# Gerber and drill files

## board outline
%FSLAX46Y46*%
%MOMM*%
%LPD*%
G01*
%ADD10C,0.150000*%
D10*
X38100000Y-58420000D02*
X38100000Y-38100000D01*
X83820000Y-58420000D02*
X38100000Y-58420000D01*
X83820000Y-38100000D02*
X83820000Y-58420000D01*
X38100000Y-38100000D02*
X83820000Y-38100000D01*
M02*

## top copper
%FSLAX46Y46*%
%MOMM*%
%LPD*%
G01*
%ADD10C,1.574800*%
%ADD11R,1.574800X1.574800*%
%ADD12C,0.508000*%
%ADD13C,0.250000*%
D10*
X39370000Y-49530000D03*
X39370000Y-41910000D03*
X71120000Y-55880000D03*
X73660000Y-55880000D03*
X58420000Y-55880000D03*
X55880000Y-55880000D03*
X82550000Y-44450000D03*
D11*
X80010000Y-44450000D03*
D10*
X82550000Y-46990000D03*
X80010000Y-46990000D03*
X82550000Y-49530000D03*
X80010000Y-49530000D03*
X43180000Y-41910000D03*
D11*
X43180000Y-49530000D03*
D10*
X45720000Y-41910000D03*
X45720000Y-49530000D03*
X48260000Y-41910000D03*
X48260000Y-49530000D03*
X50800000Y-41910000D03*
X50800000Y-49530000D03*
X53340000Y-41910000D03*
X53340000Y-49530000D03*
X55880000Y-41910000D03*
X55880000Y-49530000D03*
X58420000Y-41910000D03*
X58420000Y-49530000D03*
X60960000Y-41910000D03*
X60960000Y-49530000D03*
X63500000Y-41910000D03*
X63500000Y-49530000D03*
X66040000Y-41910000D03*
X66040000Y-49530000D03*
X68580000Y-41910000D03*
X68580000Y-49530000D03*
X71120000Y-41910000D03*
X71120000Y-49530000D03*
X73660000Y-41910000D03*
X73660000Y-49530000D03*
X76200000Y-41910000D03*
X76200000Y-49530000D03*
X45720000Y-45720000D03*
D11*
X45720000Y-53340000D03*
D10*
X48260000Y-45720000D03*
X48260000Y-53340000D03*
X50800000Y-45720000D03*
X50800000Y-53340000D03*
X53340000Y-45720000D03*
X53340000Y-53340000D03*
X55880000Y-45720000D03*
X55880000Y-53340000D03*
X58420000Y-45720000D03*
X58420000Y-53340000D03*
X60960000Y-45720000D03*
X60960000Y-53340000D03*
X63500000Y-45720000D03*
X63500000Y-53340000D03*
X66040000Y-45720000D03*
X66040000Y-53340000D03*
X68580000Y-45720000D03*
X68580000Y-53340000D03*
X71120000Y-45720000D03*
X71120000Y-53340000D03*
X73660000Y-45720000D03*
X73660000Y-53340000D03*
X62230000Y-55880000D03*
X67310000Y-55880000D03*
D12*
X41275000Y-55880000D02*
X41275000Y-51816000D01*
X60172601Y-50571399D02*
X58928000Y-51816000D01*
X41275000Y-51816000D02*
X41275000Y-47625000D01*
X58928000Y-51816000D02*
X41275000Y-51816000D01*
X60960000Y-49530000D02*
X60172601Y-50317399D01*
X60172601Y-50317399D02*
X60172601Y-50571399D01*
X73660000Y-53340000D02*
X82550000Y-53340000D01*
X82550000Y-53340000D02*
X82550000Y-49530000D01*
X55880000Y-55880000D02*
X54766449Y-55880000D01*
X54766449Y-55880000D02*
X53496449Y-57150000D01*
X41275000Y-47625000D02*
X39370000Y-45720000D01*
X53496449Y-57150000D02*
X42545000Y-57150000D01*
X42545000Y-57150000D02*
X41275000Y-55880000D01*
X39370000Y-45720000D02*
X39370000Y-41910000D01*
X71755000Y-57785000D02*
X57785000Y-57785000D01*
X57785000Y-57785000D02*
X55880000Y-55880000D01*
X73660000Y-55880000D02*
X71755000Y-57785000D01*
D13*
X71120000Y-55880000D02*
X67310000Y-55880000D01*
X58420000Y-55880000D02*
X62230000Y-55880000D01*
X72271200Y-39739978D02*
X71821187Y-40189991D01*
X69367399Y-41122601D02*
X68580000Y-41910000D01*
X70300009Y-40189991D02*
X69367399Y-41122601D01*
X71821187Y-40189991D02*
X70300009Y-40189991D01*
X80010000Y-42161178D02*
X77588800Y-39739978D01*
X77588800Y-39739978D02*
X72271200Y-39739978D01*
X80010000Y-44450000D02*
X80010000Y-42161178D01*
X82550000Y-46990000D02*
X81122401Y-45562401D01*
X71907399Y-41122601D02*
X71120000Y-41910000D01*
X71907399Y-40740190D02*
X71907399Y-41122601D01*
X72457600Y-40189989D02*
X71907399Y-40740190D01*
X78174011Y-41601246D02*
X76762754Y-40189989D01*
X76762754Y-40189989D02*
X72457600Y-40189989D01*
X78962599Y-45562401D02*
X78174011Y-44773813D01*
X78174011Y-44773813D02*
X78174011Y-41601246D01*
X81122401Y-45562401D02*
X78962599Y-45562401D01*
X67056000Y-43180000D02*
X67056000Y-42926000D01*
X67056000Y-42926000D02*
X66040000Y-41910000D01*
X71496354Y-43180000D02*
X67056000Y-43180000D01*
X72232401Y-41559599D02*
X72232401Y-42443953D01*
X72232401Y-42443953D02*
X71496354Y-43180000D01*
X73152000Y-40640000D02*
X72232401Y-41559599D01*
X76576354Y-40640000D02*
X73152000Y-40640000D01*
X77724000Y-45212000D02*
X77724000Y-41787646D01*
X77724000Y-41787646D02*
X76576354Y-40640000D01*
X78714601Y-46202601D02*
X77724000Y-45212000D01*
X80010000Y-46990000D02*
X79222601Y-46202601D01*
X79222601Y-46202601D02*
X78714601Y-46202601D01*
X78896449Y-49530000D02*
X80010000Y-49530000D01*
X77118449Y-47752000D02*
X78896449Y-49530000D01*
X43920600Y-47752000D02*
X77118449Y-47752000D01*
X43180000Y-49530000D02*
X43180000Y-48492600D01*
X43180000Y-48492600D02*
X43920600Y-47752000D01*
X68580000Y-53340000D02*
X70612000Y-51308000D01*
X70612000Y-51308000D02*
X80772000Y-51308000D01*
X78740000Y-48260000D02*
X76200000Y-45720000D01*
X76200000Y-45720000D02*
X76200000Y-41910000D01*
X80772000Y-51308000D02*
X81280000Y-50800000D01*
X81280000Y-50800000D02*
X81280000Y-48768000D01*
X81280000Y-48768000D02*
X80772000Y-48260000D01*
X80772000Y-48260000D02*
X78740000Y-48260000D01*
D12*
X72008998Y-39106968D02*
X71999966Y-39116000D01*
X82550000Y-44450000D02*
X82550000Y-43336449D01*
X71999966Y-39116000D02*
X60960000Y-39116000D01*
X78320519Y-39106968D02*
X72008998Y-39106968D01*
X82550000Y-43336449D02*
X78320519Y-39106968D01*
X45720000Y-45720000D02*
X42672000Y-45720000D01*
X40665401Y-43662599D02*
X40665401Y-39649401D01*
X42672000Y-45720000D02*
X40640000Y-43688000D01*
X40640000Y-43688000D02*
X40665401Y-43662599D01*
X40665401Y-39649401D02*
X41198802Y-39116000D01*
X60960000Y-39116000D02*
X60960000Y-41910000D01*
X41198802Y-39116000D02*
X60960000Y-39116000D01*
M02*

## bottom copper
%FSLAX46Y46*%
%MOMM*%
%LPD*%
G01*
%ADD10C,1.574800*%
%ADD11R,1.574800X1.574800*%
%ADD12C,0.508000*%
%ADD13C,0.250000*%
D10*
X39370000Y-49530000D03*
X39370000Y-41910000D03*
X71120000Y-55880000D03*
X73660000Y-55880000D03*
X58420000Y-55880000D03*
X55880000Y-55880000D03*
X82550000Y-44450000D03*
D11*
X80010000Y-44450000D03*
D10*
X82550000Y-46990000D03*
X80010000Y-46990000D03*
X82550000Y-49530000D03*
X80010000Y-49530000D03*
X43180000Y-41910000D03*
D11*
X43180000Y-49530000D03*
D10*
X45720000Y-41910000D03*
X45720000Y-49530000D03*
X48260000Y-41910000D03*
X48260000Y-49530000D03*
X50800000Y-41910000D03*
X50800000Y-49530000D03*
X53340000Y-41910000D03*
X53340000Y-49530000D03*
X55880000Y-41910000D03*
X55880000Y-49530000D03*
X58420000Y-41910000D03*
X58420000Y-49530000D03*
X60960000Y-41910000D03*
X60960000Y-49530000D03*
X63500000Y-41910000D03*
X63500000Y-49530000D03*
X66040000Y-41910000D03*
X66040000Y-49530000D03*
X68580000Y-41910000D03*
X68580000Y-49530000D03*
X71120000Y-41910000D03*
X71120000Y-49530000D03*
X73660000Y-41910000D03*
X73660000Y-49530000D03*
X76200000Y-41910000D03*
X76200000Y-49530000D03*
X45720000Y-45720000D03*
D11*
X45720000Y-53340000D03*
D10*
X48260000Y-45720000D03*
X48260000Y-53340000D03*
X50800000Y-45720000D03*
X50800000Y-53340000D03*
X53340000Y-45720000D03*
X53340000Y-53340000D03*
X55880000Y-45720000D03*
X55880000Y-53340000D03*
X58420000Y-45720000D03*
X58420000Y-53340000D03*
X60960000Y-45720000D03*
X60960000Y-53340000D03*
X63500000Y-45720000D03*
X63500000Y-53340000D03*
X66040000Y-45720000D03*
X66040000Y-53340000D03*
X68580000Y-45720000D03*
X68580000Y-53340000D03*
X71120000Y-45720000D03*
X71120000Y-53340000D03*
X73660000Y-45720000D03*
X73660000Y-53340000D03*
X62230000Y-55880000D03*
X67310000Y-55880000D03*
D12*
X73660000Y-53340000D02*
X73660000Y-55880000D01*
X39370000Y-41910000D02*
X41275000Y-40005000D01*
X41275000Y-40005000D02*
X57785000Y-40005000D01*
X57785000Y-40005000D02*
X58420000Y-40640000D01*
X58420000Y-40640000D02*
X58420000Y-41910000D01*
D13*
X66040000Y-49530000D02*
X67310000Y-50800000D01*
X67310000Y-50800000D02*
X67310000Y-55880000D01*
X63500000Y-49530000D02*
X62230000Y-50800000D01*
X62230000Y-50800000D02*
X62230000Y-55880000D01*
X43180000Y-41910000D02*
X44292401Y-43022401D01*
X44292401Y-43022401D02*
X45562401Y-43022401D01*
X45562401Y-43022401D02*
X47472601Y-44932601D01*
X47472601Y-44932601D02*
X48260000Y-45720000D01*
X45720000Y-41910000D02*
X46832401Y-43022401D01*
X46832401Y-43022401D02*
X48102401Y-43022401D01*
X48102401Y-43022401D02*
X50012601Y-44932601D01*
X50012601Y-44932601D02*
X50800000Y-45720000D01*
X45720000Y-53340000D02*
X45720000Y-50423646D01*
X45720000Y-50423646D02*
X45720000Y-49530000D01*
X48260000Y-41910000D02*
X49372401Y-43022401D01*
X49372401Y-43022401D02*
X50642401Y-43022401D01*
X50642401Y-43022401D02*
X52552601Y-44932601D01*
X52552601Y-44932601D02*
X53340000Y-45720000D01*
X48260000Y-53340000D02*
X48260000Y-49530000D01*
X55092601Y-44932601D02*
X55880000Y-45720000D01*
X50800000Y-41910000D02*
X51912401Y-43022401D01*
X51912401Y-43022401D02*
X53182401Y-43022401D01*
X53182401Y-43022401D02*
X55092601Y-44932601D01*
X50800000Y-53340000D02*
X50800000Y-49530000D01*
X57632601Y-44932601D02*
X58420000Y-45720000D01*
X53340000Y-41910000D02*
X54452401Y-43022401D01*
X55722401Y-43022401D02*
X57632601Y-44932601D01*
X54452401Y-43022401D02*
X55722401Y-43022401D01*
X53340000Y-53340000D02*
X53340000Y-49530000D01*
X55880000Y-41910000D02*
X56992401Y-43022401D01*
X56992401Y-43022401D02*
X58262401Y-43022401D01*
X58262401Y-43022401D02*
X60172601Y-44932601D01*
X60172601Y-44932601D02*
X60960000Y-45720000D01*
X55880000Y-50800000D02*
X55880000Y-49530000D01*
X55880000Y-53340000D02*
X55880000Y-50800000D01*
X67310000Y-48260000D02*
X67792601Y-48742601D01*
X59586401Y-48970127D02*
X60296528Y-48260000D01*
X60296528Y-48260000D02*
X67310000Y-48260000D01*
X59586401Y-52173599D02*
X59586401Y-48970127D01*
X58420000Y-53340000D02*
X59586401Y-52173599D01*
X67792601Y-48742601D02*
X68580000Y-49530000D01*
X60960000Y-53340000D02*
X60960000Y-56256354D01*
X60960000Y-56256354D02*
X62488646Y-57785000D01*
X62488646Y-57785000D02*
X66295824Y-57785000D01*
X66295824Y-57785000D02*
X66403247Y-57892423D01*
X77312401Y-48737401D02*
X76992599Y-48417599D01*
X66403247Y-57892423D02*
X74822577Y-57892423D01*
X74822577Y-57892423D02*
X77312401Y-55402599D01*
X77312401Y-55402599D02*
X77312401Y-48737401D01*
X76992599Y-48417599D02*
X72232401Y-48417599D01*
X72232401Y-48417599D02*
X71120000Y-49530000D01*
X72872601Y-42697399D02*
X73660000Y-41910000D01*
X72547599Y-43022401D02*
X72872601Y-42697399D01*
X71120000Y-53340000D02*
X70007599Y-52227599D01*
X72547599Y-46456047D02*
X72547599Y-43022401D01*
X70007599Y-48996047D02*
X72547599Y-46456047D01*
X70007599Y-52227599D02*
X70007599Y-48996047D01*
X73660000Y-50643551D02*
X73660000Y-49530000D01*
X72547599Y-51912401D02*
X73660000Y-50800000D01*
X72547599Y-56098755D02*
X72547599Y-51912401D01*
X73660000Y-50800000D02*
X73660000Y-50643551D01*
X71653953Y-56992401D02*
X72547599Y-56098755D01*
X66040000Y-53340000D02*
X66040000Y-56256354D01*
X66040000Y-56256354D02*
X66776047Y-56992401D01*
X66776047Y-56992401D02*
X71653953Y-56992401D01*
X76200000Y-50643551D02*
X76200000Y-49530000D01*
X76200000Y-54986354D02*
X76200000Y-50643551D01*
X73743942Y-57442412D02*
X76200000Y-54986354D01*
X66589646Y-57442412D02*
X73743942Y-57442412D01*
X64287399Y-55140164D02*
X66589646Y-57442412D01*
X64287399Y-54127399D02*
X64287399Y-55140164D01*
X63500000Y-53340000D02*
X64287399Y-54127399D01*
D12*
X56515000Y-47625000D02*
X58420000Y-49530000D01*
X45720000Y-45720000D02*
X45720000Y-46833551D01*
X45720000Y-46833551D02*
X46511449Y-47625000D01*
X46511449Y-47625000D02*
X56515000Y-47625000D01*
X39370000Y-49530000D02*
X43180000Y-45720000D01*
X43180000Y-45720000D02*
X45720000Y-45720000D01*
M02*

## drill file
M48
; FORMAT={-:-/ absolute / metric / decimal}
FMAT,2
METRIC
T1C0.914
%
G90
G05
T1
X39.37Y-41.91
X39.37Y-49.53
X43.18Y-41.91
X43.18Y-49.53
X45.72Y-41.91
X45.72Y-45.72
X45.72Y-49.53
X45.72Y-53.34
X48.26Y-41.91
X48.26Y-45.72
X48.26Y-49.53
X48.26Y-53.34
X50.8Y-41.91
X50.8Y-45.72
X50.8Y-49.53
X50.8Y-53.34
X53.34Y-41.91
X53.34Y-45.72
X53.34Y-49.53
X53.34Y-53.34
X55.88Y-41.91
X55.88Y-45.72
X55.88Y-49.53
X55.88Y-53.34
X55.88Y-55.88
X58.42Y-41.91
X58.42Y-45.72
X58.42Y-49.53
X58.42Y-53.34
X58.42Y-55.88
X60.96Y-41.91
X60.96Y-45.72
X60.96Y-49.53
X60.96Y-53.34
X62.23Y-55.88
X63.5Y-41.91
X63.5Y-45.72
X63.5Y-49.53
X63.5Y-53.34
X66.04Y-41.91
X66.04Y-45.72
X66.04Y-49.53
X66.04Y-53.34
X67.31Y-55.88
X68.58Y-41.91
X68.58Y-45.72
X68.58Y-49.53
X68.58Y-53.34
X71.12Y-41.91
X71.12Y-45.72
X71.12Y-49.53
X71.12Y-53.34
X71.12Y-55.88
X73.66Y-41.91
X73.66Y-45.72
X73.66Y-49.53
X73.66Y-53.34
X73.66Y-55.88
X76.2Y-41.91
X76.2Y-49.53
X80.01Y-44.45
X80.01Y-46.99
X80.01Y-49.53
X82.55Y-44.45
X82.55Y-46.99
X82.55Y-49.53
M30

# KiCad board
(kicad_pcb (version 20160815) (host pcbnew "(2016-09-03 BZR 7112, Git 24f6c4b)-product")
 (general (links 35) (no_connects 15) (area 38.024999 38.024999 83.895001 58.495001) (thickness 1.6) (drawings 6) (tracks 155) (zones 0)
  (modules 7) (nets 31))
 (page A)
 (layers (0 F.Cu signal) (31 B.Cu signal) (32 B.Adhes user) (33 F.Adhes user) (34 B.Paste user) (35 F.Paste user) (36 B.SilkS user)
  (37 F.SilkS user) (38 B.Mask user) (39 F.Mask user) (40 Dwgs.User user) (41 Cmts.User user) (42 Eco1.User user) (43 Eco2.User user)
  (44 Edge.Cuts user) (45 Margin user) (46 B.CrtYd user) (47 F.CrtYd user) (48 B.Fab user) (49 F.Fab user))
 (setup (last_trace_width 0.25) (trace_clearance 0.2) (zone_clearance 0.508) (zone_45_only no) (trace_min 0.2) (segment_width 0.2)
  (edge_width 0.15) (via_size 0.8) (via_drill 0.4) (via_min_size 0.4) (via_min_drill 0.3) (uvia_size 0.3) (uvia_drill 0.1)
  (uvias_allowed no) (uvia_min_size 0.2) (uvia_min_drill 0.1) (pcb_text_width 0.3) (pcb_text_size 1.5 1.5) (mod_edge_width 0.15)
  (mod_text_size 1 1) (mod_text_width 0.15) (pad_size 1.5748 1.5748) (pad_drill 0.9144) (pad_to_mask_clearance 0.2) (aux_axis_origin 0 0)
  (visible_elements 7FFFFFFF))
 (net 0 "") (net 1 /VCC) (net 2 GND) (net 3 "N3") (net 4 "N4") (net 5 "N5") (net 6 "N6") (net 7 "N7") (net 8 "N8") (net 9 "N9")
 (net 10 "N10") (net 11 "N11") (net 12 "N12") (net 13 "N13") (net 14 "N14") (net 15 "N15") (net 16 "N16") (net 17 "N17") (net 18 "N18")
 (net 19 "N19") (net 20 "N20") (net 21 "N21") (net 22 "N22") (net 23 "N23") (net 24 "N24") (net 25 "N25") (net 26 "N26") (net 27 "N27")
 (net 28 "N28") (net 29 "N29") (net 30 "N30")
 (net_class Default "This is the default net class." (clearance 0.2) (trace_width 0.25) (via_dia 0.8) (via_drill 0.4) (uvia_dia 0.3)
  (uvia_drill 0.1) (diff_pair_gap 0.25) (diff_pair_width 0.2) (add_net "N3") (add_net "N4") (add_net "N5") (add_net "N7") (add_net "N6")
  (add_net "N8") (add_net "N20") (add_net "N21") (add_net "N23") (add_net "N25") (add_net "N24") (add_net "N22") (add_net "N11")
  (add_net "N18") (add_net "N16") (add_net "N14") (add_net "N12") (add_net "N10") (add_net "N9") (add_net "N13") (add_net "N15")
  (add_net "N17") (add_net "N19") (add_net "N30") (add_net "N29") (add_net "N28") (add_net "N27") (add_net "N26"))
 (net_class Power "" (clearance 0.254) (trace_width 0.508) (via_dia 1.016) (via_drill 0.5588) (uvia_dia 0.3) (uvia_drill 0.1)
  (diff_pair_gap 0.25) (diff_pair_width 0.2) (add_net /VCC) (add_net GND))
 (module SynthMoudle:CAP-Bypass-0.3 (layer F.Cu) (at 39.37 45.72 90)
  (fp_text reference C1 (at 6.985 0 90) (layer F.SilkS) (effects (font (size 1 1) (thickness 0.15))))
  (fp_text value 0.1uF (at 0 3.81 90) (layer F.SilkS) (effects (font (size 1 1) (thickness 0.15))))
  (pad 1 thru_hole circle (at -3.81 0 90) (size 1.5748 1.5748) (drill 0.9144) (layers *.Cu *.Mask F.SilkS) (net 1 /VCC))
  (pad 2 thru_hole circle (at 3.81 0 90) (size 1.5748 1.5748) (drill 0.9144) (layers *.Cu *.Mask F.SilkS) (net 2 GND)))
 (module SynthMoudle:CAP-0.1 (layer F.Cu) (at 72.39 55.88)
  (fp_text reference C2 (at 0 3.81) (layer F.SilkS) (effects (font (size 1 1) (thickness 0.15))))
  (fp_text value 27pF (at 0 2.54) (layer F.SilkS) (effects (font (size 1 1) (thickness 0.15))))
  (pad 1 thru_hole circle (at -1.27 0) (size 1.5748 1.5748) (drill 0.9144) (layers *.Cu *.Mask F.SilkS) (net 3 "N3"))
  (pad 2 thru_hole circle (at 1.27 0) (size 1.5748 1.5748) (drill 0.9144) (layers *.Cu *.Mask F.SilkS) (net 2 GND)))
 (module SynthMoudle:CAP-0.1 (layer F.Cu) (at 57.15 55.88 180)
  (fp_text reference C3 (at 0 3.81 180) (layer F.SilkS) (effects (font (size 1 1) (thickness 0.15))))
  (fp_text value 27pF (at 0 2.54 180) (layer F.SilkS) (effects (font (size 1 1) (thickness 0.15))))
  (pad 1 thru_hole circle (at -1.27 0 180) (size 1.5748 1.5748) (drill 0.9144) (layers *.Cu *.Mask F.SilkS) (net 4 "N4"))
  (pad 2 thru_hole circle (at 1.27 0 180) (size 1.5748 1.5748) (drill 0.9144) (layers *.Cu *.Mask F.SilkS) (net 2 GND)))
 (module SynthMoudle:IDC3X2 (layer F.Cu) (at 81.28 46.99 270)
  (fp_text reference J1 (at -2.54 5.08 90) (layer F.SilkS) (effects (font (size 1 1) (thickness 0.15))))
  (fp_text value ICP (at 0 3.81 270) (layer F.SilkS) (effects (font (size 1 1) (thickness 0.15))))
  (pad 2 thru_hole circle (at -2.54 -1.27 270) (size 1.5748 1.5748) (drill 0.9144) (layers *.Cu *.Mask) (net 1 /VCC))
  (pad 1 thru_hole rect (at -2.54 1.27 270) (size 1.5748 1.5748) (drill 0.9144) (layers *.Cu *.Mask) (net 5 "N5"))
  (pad 4 thru_hole circle (at 0 -1.27 270) (size 1.5748 1.5748) (drill 0.9144) (layers *.Cu *.Mask) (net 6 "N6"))
  (pad 3 thru_hole circle (at 0 1.27 270) (size 1.5748 1.5748) (drill 0.9144) (layers *.Cu *.Mask) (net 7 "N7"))
  (pad 6 thru_hole circle (at 2.54 -1.27 270) (size 1.5748 1.5748) (drill 0.9144) (layers *.Cu *.Mask) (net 2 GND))
  (pad 5 thru_hole circle (at 2.54 1.27 270) (size 1.5748 1.5748) (drill 0.9144) (layers *.Cu *.Mask) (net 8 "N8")))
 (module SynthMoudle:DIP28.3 (layer F.Cu) (at 59.69 45.72)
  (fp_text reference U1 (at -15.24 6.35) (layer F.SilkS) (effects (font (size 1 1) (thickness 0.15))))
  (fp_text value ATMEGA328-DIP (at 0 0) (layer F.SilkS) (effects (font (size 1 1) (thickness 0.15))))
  (pad 28 thru_hole circle (at -16.51 -3.81) (size 1.5748 1.5748) (drill 0.9144) (layers *.Cu *.Mask) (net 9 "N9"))
  (pad 1 thru_hole rect (at -16.51 3.81) (size 1.5748 1.5748) (drill 0.9144) (layers *.Cu *.Mask) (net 8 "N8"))
  (pad 27 thru_hole circle (at -13.97 -3.81) (size 1.5748 1.5748) (drill 0.9144) (layers *.Cu *.Mask) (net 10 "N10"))
  (pad 2 thru_hole circle (at -13.97 3.81) (size 1.5748 1.5748) (drill 0.9144) (layers *.Cu *.Mask) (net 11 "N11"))
  (pad 26 thru_hole circle (at -11.43 -3.81) (size 1.5748 1.5748) (drill 0.9144) (layers *.Cu *.Mask) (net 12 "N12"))
  (pad 3 thru_hole circle (at -11.43 3.81) (size 1.5748 1.5748) (drill 0.9144) (layers *.Cu *.Mask) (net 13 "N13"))
  (pad 25 thru_hole circle (at -8.89 -3.81) (size 1.5748 1.5748) (drill 0.9144) (layers *.Cu *.Mask) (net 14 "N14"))
  (pad 4 thru_hole circle (at -8.89 3.81) (size 1.5748 1.5748) (drill 0.9144) (layers *.Cu *.Mask) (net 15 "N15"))
  (pad 24 thru_hole circle (at -6.35 -3.81) (size 1.5748 1.5748) (drill 0.9144) (layers *.Cu *.Mask) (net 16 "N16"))
  (pad 5 thru_hole circle (at -6.35 3.81) (size 1.5748 1.5748) (drill 0.9144) (layers *.Cu *.Mask) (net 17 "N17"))
  (pad 23 thru_hole circle (at -3.81 -3.81) (size 1.5748 1.5748) (drill 0.9144) (layers *.Cu *.Mask) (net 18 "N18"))
  (pad 6 thru_hole circle (at -3.81 3.81) (size 1.5748 1.5748) (drill 0.9144) (layers *.Cu *.Mask) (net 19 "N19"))
  (pad 22 thru_hole circle (at -1.27 -3.81) (size 1.5748 1.5748) (drill 0.9144) (layers *.Cu *.Mask) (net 2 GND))
  (pad 7 thru_hole circle (at -1.27 3.81) (size 1.5748 1.5748) (drill 0.9144) (layers *.Cu *.Mask) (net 1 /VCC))
  (pad 21 thru_hole circle (at 1.27 -3.81) (size 1.5748 1.5748) (drill 0.9144) (layers *.Cu *.Mask) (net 1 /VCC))
  (pad 8 thru_hole circle (at 1.27 3.81) (size 1.5748 1.5748) (drill 0.9144) (layers *.Cu *.Mask) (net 2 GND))
  (pad 20 thru_hole circle (at 3.81 -3.81) (size 1.5748 1.5748) (drill 0.9144) (layers *.Cu *.Mask))
  (pad 9 thru_hole circle (at 3.81 3.81) (size 1.5748 1.5748) (drill 0.9144) (layers *.Cu *.Mask) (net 4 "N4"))
  (pad 19 thru_hole circle (at 6.35 -3.81) (size 1.5748 1.5748) (drill 0.9144) (layers *.Cu *.Mask) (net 7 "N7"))
  (pad 10 thru_hole circle (at 6.35 3.81) (size 1.5748 1.5748) (drill 0.9144) (layers *.Cu *.Mask) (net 3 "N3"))
  (pad 18 thru_hole circle (at 8.89 -3.81) (size 1.5748 1.5748) (drill 0.9144) (layers *.Cu *.Mask) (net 5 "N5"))
  (pad 11 thru_hole circle (at 8.89 3.81) (size 1.5748 1.5748) (drill 0.9144) (layers *.Cu *.Mask) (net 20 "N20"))
  (pad 17 thru_hole circle (at 11.43 -3.81) (size 1.5748 1.5748) (drill 0.9144) (layers *.Cu *.Mask) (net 6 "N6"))
  (pad 12 thru_hole circle (at 11.43 3.81) (size 1.5748 1.5748) (drill 0.9144) (layers *.Cu *.Mask) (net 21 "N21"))
  (pad 16 thru_hole circle (at 13.97 -3.81) (size 1.5748 1.5748) (drill 0.9144) (layers *.Cu *.Mask) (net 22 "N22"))
  (pad 13 thru_hole circle (at 13.97 3.81) (size 1.5748 1.5748) (drill 0.9144) (layers *.Cu *.Mask) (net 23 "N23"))
  (pad 15 thru_hole circle (at 16.51 -3.81) (size 1.5748 1.5748) (drill 0.9144) (layers *.Cu *.Mask) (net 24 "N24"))
  (pad 14 thru_hole circle (at 16.51 3.81) (size 1.5748 1.5748) (drill 0.9144) (layers *.Cu *.Mask) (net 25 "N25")))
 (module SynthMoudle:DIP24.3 (layer F.Cu) (at 59.69 49.53)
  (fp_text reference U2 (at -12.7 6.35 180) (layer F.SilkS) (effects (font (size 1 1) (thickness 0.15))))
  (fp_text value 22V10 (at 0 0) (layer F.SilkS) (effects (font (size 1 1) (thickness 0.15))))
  (pad 24 thru_hole circle (at -13.97 -3.81) (size 1.5748 1.5748) (drill 0.9144) (layers *.Cu *.Mask) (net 1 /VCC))
  (pad 1 thru_hole rect (at -13.97 3.81) (size 1.5748 1.5748) (drill 0.9144) (layers *.Cu *.Mask) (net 11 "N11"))
  (pad 23 thru_hole circle (at -11.43 -3.81) (size 1.5748 1.5748) (drill 0.9144) (layers *.Cu *.Mask) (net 9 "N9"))
  (pad 2 thru_hole circle (at -11.43 3.81) (size 1.5748 1.5748) (drill 0.9144) (layers *.Cu *.Mask) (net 13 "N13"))
  (pad 22 thru_hole circle (at -8.89 -3.81) (size 1.5748 1.5748) (drill 0.9144) (layers *.Cu *.Mask) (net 10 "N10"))
  (pad 3 thru_hole circle (at -8.89 3.81) (size 1.5748 1.5748) (drill 0.9144) (layers *.Cu *.Mask) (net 15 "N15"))
  (pad 21 thru_hole circle (at -6.35 -3.81) (size 1.5748 1.5748) (drill 0.9144) (layers *.Cu *.Mask) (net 12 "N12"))
  (pad 4 thru_hole circle (at -6.35 3.81) (size 1.5748 1.5748) (drill 0.9144) (layers *.Cu *.Mask) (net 17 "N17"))
  (pad 20 thru_hole circle (at -3.81 -3.81) (size 1.5748 1.5748) (drill 0.9144) (layers *.Cu *.Mask) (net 14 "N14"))
  (pad 5 thru_hole circle (at -3.81 3.81) (size 1.5748 1.5748) (drill 0.9144) (layers *.Cu *.Mask) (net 19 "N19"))
  (pad 19 thru_hole circle (at -1.27 -3.81) (size 1.5748 1.5748) (drill 0.9144) (layers *.Cu *.Mask) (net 16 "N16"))
  (pad 6 thru_hole circle (at -1.27 3.81) (size 1.5748 1.5748) (drill 0.9144) (layers *.Cu *.Mask) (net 20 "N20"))
  (pad 18 thru_hole circle (at 1.27 -3.81) (size 1.5748 1.5748) (drill 0.9144) (layers *.Cu *.Mask) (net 18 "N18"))
  (pad 7 thru_hole circle (at 1.27 3.81) (size 1.5748 1.5748) (drill 0.9144) (layers *.Cu *.Mask) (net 21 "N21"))
  (pad 17 thru_hole circle (at 3.81 -3.81) (size 1.5748 1.5748) (drill 0.9144) (layers *.Cu *.Mask) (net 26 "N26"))
  (pad 8 thru_hole circle (at 3.81 3.81) (size 1.5748 1.5748) (drill 0.9144) (layers *.Cu *.Mask) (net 25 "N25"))
  (pad 16 thru_hole circle (at 6.35 -3.81) (size 1.5748 1.5748) (drill 0.9144) (layers *.Cu *.Mask) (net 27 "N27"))
  (pad 9 thru_hole circle (at 6.35 3.81) (size 1.5748 1.5748) (drill 0.9144) (layers *.Cu *.Mask) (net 23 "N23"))
  (pad 15 thru_hole circle (at 8.89 -3.81) (size 1.5748 1.5748) (drill 0.9144) (layers *.Cu *.Mask) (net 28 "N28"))
  (pad 10 thru_hole circle (at 8.89 3.81) (size 1.5748 1.5748) (drill 0.9144) (layers *.Cu *.Mask) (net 24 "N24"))
  (pad 14 thru_hole circle (at 11.43 -3.81) (size 1.5748 1.5748) (drill 0.9144) (layers *.Cu *.Mask) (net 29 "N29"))
  (pad 11 thru_hole circle (at 11.43 3.81) (size 1.5748 1.5748) (drill 0.9144) (layers *.Cu *.Mask) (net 22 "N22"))
  (pad 13 thru_hole circle (at 13.97 -3.81) (size 1.5748 1.5748) (drill 0.9144) (layers *.Cu *.Mask) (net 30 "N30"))
  (pad 12 thru_hole circle (at 13.97 3.81) (size 1.5748 1.5748) (drill 0.9144) (layers *.Cu *.Mask) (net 2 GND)))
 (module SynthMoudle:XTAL (layer F.Cu) (at 64.77 55.88)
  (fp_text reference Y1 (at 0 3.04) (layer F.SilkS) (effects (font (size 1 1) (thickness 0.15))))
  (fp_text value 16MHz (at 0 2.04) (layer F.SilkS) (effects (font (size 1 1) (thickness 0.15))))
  (pad 1 thru_hole circle (at -2.54 0) (size 1.5748 1.5748) (drill 0.9144) (layers *.Cu *.Mask F.SilkS) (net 4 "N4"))
  (pad 2 thru_hole circle (at 2.54 0) (size 1.5748 1.5748) (drill 0.9144) (layers *.Cu *.Mask F.SilkS) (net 3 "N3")))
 (gr_line (start 38.1 58.42) (end 38.1 38.1) (angle 90) (layer Edge.Cuts) (width 0.15))
 (gr_line (start 83.82 58.42) (end 38.1 58.42) (angle 90) (layer Edge.Cuts) (width 0.15))
 (gr_line (start 83.82 38.1) (end 83.82 58.42) (angle 90) (layer Edge.Cuts) (width 0.15))
 (gr_line (start 38.1 38.1) (end 83.82 38.1) (angle 90) (layer Edge.Cuts) (width 0.15))
 (segment (start 41.275 55.88) (end 41.275 51.816) (width 0.508) (layer F.Cu) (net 2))
 (segment (start 60.172601 50.571399) (end 58.928 51.816) (width 0.508) (layer F.Cu) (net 2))
 (segment (start 41.275 51.816) (end 41.275 47.625) (width 0.508) (layer F.Cu) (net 2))
 (segment (start 58.928 51.816) (end 41.275 51.816) (width 0.508) (layer F.Cu) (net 2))
 (segment (start 60.96 49.53) (end 60.172601 50.317399) (width 0.508) (layer F.Cu) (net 2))
 (segment (start 60.172601 50.317399) (end 60.172601 50.571399) (width 0.508) (layer F.Cu) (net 2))
 (segment (start 73.66 53.34) (end 82.55 53.34) (width 0.508) (layer F.Cu) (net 2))
 (segment (start 82.55 53.34) (end 82.55 49.53) (width 0.508) (layer F.Cu) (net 2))
 (segment (start 55.88 55.88) (end 54.766449 55.88) (width 0.508) (layer F.Cu) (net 2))
 (segment (start 54.766449 55.88) (end 53.496449 57.15) (width 0.508) (layer F.Cu) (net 2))
 (segment (start 41.275 47.625) (end 39.37 45.72) (width 0.508) (layer F.Cu) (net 2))
 (segment (start 53.496449 57.15) (end 42.545 57.15) (width 0.508) (layer F.Cu) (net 2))
 (segment (start 42.545 57.15) (end 41.275 55.88) (width 0.508) (layer F.Cu) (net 2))
 (segment (start 39.37 45.72) (end 39.37 41.91) (width 0.508) (layer F.Cu) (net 2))
 (segment (start 71.755 57.785) (end 57.785 57.785) (width 0.508) (layer F.Cu) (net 2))
 (segment (start 57.785 57.785) (end 55.88 55.88) (width 0.508) (layer F.Cu) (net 2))
 (segment (start 73.66 55.88) (end 71.755 57.785) (width 0.508) (layer F.Cu) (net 2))
 (segment (start 73.66 53.34) (end 73.66 55.88) (width 0.508) (layer B.Cu) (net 2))
 (segment (start 39.37 41.91) (end 41.275 40.005) (width 0.508) (layer B.Cu) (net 2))
 (segment (start 41.275 40.005) (end 57.785 40.005) (width 0.508) (layer B.Cu) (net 2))
 (segment (start 57.785 40.005) (end 58.42 40.64) (width 0.508) (layer B.Cu) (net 2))
 (segment (start 58.42 40.64) (end 58.42 41.91) (width 0.508) (layer B.Cu) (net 2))
 (segment (start 66.04 49.53) (end 67.31 50.8) (width 0.25) (layer B.Cu) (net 3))
 (segment (start 67.31 50.8) (end 67.31 55.88) (width 0.25) (layer B.Cu) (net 3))
 (segment (start 71.12 55.88) (end 67.31 55.88) (width 0.25) (layer F.Cu) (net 3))
 (segment (start 63.5 49.53) (end 62.23 50.8) (width 0.25) (layer B.Cu) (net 4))
 (segment (start 62.23 50.8) (end 62.23 55.88) (width 0.25) (layer B.Cu) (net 4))
 (segment (start 58.42 55.88) (end 62.23 55.88) (width 0.25) (layer F.Cu) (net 4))
 (segment (start 72.2712 39.739978) (end 71.821187 40.189991) (width 0.25) (layer F.Cu) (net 5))
 (segment (start 69.367399 41.122601) (end 68.58 41.91) (width 0.25) (layer F.Cu) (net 5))
 (segment (start 70.300009 40.189991) (end 69.367399 41.122601) (width 0.25) (layer F.Cu) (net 5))
 (segment (start 71.821187 40.189991) (end 70.300009 40.189991) (width 0.25) (layer F.Cu) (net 5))
 (segment (start 80.01 42.161178) (end 77.5888 39.739978) (width 0.25) (layer F.Cu) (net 5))
 (segment (start 77.5888 39.739978) (end 72.2712 39.739978) (width 0.25) (layer F.Cu) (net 5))
 (segment (start 80.01 44.45) (end 80.01 42.161178) (width 0.25) (layer F.Cu) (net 5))
 (segment (start 82.55 46.99) (end 81.122401 45.562401) (width 0.25) (layer F.Cu) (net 6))
 (segment (start 71.907399 41.122601) (end 71.12 41.91) (width 0.25) (layer F.Cu) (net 6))
 (segment (start 71.907399 40.74019) (end 71.907399 41.122601) (width 0.25) (layer F.Cu) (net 6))
 (segment (start 72.4576 40.189989) (end 71.907399 40.74019) (width 0.25) (layer F.Cu) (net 6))
 (segment (start 78.174011 41.601246) (end 76.762754 40.189989) (width 0.25) (layer F.Cu) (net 6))
 (segment (start 76.762754 40.189989) (end 72.4576 40.189989) (width 0.25) (layer F.Cu) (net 6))
 (segment (start 78.962599 45.562401) (end 78.174011 44.773813) (width 0.25) (layer F.Cu) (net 6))
 (segment (start 78.174011 44.773813) (end 78.174011 41.601246) (width 0.25) (layer F.Cu) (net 6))
 (segment (start 81.122401 45.562401) (end 78.962599 45.562401) (width 0.25) (layer F.Cu) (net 6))
 (segment (start 67.056 43.18) (end 67.056 42.926) (width 0.25) (layer F.Cu) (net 7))
 (segment (start 67.056 42.926) (end 66.04 41.91) (width 0.25) (layer F.Cu) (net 7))
 (segment (start 71.496354 43.18) (end 67.056 43.18) (width 0.25) (layer F.Cu) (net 7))
 (segment (start 72.232401 41.559599) (end 72.232401 42.443953) (width 0.25) (layer F.Cu) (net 7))
 (segment (start 72.232401 42.443953) (end 71.496354 43.18) (width 0.25) (layer F.Cu) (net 7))
 (segment (start 73.152 40.64) (end 72.232401 41.559599) (width 0.25) (layer F.Cu) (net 7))
 (segment (start 76.576354 40.64) (end 73.152 40.64) (width 0.25) (layer F.Cu) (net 7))
 (segment (start 77.724 45.212) (end 77.724 41.787646) (width 0.25) (layer F.Cu) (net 7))
 (segment (start 77.724 41.787646) (end 76.576354 40.64) (width 0.25) (layer F.Cu) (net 7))
 (segment (start 78.714601 46.202601) (end 77.724 45.212) (width 0.25) (layer F.Cu) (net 7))
 (segment (start 80.01 46.99) (end 79.222601 46.202601) (width 0.25) (layer F.Cu) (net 7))
 (segment (start 79.222601 46.202601) (end 78.714601 46.202601) (width 0.25) (layer F.Cu) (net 7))
 (segment (start 78.896449 49.53) (end 80.01 49.53) (width 0.25) (layer F.Cu) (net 8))
 (segment (start 77.118449 47.752) (end 78.896449 49.53) (width 0.25) (layer F.Cu) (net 8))
 (segment (start 43.9206 47.752) (end 77.118449 47.752) (width 0.25) (layer F.Cu) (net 8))
 (segment (start 43.18 49.53) (end 43.18 48.4926) (width 0.25) (layer F.Cu) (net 8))
 (segment (start 43.18 48.4926) (end 43.9206 47.752) (width 0.25) (layer F.Cu) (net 8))
 (segment (start 43.18 41.91) (end 44.292401 43.022401) (width 0.25) (layer B.Cu) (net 9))
 (segment (start 44.292401 43.022401) (end 45.562401 43.022401) (width 0.25) (layer B.Cu) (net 9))
 (segment (start 45.562401 43.022401) (end 47.472601 44.932601) (width 0.25) (layer B.Cu) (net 9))
 (segment (start 47.472601 44.932601) (end 48.26 45.72) (width 0.25) (layer B.Cu) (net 9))
 (segment (start 45.72 41.91) (end 46.832401 43.022401) (width 0.25) (layer B.Cu) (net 10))
 (segment (start 46.832401 43.022401) (end 48.102401 43.022401) (width 0.25) (layer B.Cu) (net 10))
 (segment (start 48.102401 43.022401) (end 50.012601 44.932601) (width 0.25) (layer B.Cu) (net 10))
 (segment (start 50.012601 44.932601) (end 50.8 45.72) (width 0.25) (layer B.Cu) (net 10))
 (segment (start 45.72 53.34) (end 45.72 50.423646) (width 0.25) (layer B.Cu) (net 11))
 (segment (start 45.72 50.423646) (end 45.72 49.53) (width 0.25) (layer B.Cu) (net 11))
 (segment (start 48.26 41.91) (end 49.372401 43.022401) (width 0.25) (layer B.Cu) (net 12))
 (segment (start 49.372401 43.022401) (end 50.642401 43.022401) (width 0.25) (layer B.Cu) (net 12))
 (segment (start 50.642401 43.022401) (end 52.552601 44.932601) (width 0.25) (layer B.Cu) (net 12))
 (segment (start 52.552601 44.932601) (end 53.34 45.72) (width 0.25) (layer B.Cu) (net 12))
 (segment (start 48.26 53.34) (end 48.26 49.53) (width 0.25) (layer B.Cu) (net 13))
 (segment (start 55.092601 44.932601) (end 55.88 45.72) (width 0.25) (layer B.Cu) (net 14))
 (segment (start 50.8 41.91) (end 51.912401 43.022401) (width 0.25) (layer B.Cu) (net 14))
 (segment (start 51.912401 43.022401) (end 53.182401 43.022401) (width 0.25) (layer B.Cu) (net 14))
 (segment (start 53.182401 43.022401) (end 55.092601 44.932601) (width 0.25) (layer B.Cu) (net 14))
 (segment (start 50.8 53.34) (end 50.8 49.53) (width 0.25) (layer B.Cu) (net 15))
 (segment (start 57.632601 44.932601) (end 58.42 45.72) (width 0.25) (layer B.Cu) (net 16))
 (segment (start 53.34 41.91) (end 54.452401 43.022401) (width 0.25) (layer B.Cu) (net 16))
 (segment (start 55.722401 43.022401) (end 57.632601 44.932601) (width 0.25) (layer B.Cu) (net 16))
 (segment (start 54.452401 43.022401) (end 55.722401 43.022401) (width 0.25) (layer B.Cu) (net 16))
 (segment (start 53.34 53.34) (end 53.34 49.53) (width 0.25) (layer B.Cu) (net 17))
 (segment (start 55.88 41.91) (end 56.992401 43.022401) (width 0.25) (layer B.Cu) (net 18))
 (segment (start 56.992401 43.022401) (end 58.262401 43.022401) (width 0.25) (layer B.Cu) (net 18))
 (segment (start 58.262401 43.022401) (end 60.172601 44.932601) (width 0.25) (layer B.Cu) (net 18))
 (segment (start 60.172601 44.932601) (end 60.96 45.72) (width 0.25) (layer B.Cu) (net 18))
 (segment (start 55.88 50.8) (end 55.88 49.53) (width 0.25) (layer B.Cu) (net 19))
 (segment (start 55.88 53.34) (end 55.88 50.8) (width 0.25) (layer B.Cu) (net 19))
 (segment (start 67.31 48.26) (end 67.792601 48.742601) (width 0.25) (layer B.Cu) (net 20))
 (segment (start 59.586401 48.970127) (end 60.296528 48.26) (width 0.25) (layer B.Cu) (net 20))
 (segment (start 60.296528 48.26) (end 67.31 48.26) (width 0.25) (layer B.Cu) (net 20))
 (segment (start 59.586401 52.173599) (end 59.586401 48.970127) (width 0.25) (layer B.Cu) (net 20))
 (segment (start 58.42 53.34) (end 59.586401 52.173599) (width 0.25) (layer B.Cu) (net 20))
 (segment (start 67.792601 48.742601) (end 68.58 49.53) (width 0.25) (layer B.Cu) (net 20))
 (segment (start 60.96 53.34) (end 60.96 56.256354) (width 0.25) (layer B.Cu) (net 21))
 (segment (start 60.96 56.256354) (end 62.488646 57.785) (width 0.25) (layer B.Cu) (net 21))
 (segment (start 62.488646 57.785) (end 66.295824 57.785) (width 0.25) (layer B.Cu) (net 21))
 (segment (start 66.295824 57.785) (end 66.403247 57.892423) (width 0.25) (layer B.Cu) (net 21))
 (segment (start 77.312401 48.737401) (end 76.992599 48.417599) (width 0.25) (layer B.Cu) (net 21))
 (segment (start 66.403247 57.892423) (end 74.822577 57.892423) (width 0.25) (layer B.Cu) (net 21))
 (segment (start 74.822577 57.892423) (end 77.312401 55.402599) (width 0.25) (layer B.Cu) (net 21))
 (segment (start 77.312401 55.402599) (end 77.312401 48.737401) (width 0.25) (layer B.Cu) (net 21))
 (segment (start 76.992599 48.417599) (end 72.232401 48.417599) (width 0.25) (layer B.Cu) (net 21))
 (segment (start 72.232401 48.417599) (end 71.12 49.53) (width 0.25) (layer B.Cu) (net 21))
 (segment (start 72.872601 42.697399) (end 73.66 41.91) (width 0.25) (layer B.Cu) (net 22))
 (segment (start 72.547599 43.022401) (end 72.872601 42.697399) (width 0.25) (layer B.Cu) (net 22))
 (segment (start 71.12 53.34) (end 70.007599 52.227599) (width 0.25) (layer B.Cu) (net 22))
 (segment (start 72.547599 46.456047) (end 72.547599 43.022401) (width 0.25) (layer B.Cu) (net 22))
 (segment (start 70.007599 48.996047) (end 72.547599 46.456047) (width 0.25) (layer B.Cu) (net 22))
 (segment (start 70.007599 52.227599) (end 70.007599 48.996047) (width 0.25) (layer B.Cu) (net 22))
 (segment (start 73.66 50.643551) (end 73.66 49.53) (width 0.25) (layer B.Cu) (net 23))
 (segment (start 72.547599 51.912401) (end 73.66 50.8) (width 0.25) (layer B.Cu) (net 23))
 (segment (start 72.547599 56.098755) (end 72.547599 51.912401) (width 0.25) (layer B.Cu) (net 23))
 (segment (start 73.66 50.8) (end 73.66 50.643551) (width 0.25) (layer B.Cu) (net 23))
 (segment (start 71.653953 56.992401) (end 72.547599 56.098755) (width 0.25) (layer B.Cu) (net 23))
 (segment (start 66.04 53.34) (end 66.04 56.256354) (width 0.25) (layer B.Cu) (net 23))
 (segment (start 66.04 56.256354) (end 66.776047 56.992401) (width 0.25) (layer B.Cu) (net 23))
 (segment (start 66.776047 56.992401) (end 71.653953 56.992401) (width 0.25) (layer B.Cu) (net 23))
 (segment (start 68.58 53.34) (end 70.612 51.308) (width 0.25) (layer F.Cu) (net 24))
 (segment (start 70.612 51.308) (end 80.772 51.308) (width 0.25) (layer F.Cu) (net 24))
 (segment (start 78.74 48.26) (end 76.2 45.72) (width 0.25) (layer F.Cu) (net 24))
 (segment (start 76.2 45.72) (end 76.2 41.91) (width 0.25) (layer F.Cu) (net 24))
 (segment (start 80.772 51.308) (end 81.28 50.8) (width 0.25) (layer F.Cu) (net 24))
 (segment (start 81.28 50.8) (end 81.28 48.768) (width 0.25) (layer F.Cu) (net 24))
 (segment (start 81.28 48.768) (end 80.772 48.26) (width 0.25) (layer F.Cu) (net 24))
 (segment (start 80.772 48.26) (end 78.74 48.26) (width 0.25) (layer F.Cu) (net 24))
 (segment (start 76.2 50.643551) (end 76.2 49.53) (width 0.25) (layer B.Cu) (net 25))
 (segment (start 76.2 54.986354) (end 76.2 50.643551) (width 0.25) (layer B.Cu) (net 25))
 (segment (start 73.743942 57.442412) (end 76.2 54.986354) (width 0.25) (layer B.Cu) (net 25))
 (segment (start 66.589646 57.442412) (end 73.743942 57.442412) (width 0.25) (layer B.Cu) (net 25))
 (segment (start 64.287399 55.140164) (end 66.589646 57.442412) (width 0.25) (layer B.Cu) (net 25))
 (segment (start 64.287399 54.127399) (end 64.287399 55.140164) (width 0.25) (layer B.Cu) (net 25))
 (segment (start 63.5 53.34) (end 64.287399 54.127399) (width 0.25) (layer B.Cu) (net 25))
 (segment (start 72.008998 39.106968) (end 71.999966 39.116) (width 0.508) (layer F.Cu) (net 1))
 (segment (start 82.55 44.45) (end 82.55 43.336449) (width 0.508) (layer F.Cu) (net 1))
 (segment (start 71.999966 39.116) (end 60.96 39.116) (width 0.508) (layer F.Cu) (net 1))
 (segment (start 78.320519 39.106968) (end 72.008998 39.106968) (width 0.508) (layer F.Cu) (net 1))
 (segment (start 82.55 43.336449) (end 78.320519 39.106968) (width 0.508) (layer F.Cu) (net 1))
 (segment (start 45.72 45.72) (end 42.672 45.72) (width 0.508) (layer F.Cu) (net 1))
 (segment (start 40.665401 43.662599) (end 40.665401 39.649401) (width 0.508) (layer F.Cu) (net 1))
 (segment (start 42.672 45.72) (end 40.64 43.688) (width 0.508) (layer F.Cu) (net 1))
 (segment (start 40.64 43.688) (end 40.665401 43.662599) (width 0.508) (layer F.Cu) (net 1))
 (segment (start 40.665401 39.649401) (end 41.198802 39.116) (width 0.508) (layer F.Cu) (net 1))
 (segment (start 60.96 39.116) (end 60.96 41.91) (width 0.508) (layer F.Cu) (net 1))
 (segment (start 41.198802 39.116) (end 60.96 39.116) (width 0.508) (layer F.Cu) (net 1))
 (segment (start 56.515 47.625) (end 58.42 49.53) (width 0.508) (layer B.Cu) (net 1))
 (segment (start 45.72 45.72) (end 45.72 46.833551) (width 0.508) (layer B.Cu) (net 1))
 (segment (start 45.72 46.833551) (end 46.511449 47.625) (width 0.508) (layer B.Cu) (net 1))
 (segment (start 46.511449 47.625) (end 56.515 47.625) (width 0.508) (layer B.Cu) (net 1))
 (segment (start 39.37 49.53) (end 43.18 45.72) (width 0.508) (layer B.Cu) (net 1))
 (segment (start 43.18 45.72) (end 45.72 45.72) (width 0.508) (layer B.Cu) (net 1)))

